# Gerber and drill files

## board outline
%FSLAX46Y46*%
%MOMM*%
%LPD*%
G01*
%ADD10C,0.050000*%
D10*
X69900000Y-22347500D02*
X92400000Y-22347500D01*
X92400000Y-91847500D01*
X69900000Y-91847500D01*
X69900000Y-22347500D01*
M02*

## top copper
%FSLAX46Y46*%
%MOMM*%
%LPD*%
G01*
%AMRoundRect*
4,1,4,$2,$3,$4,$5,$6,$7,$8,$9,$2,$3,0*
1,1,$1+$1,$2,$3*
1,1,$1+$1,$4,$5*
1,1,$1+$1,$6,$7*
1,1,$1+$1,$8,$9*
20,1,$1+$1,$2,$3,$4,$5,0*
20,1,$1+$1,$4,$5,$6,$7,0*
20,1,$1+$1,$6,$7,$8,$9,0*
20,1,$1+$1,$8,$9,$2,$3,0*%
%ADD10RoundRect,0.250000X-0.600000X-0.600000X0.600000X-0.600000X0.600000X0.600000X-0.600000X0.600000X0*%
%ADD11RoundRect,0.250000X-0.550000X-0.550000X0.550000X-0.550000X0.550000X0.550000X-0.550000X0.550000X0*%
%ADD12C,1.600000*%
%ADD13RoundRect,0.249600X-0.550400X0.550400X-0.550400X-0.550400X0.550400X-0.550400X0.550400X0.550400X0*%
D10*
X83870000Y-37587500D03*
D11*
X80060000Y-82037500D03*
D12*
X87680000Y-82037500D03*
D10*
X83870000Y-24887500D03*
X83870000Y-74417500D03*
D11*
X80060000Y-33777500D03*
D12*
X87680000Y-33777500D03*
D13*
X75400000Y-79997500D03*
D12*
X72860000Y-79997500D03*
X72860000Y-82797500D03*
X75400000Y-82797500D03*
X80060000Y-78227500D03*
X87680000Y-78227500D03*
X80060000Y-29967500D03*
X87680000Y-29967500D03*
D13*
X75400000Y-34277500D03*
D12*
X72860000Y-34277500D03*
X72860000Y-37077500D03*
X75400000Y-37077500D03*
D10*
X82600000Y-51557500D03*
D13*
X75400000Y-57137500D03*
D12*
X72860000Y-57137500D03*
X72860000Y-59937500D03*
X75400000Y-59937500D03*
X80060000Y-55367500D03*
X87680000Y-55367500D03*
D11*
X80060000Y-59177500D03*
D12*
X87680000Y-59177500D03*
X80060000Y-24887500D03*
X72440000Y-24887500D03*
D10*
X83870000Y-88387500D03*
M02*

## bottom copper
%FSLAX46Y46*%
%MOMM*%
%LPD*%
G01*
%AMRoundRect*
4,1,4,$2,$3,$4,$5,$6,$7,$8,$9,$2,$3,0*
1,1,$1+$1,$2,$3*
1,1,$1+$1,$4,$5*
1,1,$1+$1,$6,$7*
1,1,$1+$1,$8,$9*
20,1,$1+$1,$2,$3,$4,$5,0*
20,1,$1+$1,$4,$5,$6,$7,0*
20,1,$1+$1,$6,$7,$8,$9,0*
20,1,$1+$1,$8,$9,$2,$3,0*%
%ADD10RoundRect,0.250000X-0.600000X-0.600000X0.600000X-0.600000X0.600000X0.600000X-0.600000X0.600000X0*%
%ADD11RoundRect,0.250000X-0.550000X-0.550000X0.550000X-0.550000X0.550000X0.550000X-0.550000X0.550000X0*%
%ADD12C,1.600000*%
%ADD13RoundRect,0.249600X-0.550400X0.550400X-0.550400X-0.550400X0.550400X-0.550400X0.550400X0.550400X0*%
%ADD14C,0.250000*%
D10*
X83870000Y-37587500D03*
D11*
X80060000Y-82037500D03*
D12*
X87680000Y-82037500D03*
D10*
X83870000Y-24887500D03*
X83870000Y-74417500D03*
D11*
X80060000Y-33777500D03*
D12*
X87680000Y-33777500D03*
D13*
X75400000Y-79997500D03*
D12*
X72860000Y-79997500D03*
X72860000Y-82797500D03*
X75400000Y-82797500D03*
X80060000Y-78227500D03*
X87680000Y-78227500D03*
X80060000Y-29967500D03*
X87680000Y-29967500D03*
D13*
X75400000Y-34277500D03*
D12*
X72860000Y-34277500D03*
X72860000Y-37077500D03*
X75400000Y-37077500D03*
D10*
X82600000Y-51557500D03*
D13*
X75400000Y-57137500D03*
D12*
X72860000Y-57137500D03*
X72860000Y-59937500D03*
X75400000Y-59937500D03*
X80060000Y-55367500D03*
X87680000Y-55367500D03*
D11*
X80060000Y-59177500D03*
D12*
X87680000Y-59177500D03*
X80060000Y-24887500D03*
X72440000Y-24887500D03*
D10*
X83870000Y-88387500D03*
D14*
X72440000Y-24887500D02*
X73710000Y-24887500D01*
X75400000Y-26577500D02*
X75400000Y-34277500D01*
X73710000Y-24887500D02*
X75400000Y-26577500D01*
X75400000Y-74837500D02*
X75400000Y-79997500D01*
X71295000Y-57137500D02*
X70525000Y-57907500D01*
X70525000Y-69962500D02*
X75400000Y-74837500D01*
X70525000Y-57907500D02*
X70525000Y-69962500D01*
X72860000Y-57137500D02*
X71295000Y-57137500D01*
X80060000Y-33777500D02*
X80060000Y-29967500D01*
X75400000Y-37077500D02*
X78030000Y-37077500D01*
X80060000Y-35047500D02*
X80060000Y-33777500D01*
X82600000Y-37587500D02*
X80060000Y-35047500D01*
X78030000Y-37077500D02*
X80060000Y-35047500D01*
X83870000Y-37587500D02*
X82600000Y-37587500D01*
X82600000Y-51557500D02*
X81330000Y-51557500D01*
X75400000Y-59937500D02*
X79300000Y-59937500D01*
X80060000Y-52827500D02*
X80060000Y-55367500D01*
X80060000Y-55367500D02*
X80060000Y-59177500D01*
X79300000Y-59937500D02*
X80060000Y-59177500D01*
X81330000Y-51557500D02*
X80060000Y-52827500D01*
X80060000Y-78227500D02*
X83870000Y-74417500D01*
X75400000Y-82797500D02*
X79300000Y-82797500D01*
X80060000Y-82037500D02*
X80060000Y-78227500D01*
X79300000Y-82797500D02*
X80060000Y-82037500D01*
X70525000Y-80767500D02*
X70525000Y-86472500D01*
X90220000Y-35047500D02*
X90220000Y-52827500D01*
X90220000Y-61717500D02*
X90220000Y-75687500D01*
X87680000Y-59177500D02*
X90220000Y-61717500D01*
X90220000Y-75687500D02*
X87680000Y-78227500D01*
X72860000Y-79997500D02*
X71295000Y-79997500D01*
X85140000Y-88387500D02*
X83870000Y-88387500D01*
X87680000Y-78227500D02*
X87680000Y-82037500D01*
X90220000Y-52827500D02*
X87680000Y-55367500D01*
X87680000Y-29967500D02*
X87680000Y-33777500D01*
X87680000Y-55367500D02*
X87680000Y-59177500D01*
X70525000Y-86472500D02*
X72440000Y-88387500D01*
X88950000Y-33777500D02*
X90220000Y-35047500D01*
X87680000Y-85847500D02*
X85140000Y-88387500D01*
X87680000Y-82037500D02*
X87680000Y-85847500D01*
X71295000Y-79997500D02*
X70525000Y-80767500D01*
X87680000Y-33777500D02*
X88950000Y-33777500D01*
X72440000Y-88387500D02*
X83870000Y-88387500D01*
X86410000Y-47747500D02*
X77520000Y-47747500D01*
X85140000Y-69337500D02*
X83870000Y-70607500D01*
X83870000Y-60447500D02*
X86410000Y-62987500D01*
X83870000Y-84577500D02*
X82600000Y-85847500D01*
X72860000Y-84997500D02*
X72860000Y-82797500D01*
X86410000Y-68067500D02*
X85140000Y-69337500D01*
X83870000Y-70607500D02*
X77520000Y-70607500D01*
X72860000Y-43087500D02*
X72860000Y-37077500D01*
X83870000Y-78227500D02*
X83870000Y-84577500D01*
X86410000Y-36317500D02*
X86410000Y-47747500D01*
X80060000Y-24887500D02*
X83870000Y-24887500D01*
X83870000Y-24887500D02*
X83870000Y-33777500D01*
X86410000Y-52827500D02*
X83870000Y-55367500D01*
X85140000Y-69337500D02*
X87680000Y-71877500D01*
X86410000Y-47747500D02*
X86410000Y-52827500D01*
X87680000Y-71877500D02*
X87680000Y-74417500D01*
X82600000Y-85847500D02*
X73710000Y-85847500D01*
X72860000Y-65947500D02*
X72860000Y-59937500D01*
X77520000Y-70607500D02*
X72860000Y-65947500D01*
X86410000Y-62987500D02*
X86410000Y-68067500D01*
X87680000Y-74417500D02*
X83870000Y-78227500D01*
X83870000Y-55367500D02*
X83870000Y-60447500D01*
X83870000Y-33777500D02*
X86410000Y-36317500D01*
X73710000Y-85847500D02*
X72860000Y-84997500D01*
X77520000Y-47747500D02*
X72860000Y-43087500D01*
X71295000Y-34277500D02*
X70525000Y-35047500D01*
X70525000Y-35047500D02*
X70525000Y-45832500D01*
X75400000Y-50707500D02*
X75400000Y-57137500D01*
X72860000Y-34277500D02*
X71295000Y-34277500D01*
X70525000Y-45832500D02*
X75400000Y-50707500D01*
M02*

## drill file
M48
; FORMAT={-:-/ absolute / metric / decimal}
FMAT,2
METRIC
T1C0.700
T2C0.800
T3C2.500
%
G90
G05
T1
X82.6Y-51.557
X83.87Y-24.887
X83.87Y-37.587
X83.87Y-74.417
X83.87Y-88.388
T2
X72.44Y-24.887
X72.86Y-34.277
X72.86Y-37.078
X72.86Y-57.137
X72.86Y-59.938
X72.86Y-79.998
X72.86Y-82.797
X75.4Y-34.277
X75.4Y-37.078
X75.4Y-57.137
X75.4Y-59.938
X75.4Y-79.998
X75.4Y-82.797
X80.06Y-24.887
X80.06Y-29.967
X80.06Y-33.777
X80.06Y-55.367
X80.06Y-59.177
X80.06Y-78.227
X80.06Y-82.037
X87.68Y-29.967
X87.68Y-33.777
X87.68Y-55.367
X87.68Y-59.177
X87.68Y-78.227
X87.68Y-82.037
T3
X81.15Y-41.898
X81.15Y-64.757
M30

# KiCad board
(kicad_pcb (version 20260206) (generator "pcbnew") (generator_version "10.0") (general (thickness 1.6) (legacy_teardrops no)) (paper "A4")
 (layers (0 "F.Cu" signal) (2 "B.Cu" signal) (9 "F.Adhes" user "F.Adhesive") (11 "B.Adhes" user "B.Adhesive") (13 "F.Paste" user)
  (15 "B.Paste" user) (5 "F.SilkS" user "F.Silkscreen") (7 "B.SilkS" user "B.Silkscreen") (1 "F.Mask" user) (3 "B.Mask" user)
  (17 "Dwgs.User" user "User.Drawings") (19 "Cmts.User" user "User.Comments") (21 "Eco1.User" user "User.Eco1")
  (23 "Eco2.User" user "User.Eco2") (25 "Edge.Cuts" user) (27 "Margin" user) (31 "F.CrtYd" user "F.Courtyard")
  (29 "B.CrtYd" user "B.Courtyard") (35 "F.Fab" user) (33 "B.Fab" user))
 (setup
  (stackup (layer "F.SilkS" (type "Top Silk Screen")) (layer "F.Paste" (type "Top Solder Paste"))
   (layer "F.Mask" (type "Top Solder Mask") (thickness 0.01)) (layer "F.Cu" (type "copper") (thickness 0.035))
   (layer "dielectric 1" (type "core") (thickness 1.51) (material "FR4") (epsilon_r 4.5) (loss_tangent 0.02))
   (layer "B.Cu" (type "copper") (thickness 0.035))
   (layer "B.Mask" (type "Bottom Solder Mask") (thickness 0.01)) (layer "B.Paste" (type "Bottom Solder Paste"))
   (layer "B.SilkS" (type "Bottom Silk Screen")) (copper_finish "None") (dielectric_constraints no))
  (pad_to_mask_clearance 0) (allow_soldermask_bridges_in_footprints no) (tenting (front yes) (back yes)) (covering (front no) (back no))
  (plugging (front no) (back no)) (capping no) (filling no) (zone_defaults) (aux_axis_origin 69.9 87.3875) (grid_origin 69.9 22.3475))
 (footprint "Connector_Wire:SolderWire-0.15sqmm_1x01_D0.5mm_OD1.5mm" (layer "F.Cu") (at 83.87 37.5875)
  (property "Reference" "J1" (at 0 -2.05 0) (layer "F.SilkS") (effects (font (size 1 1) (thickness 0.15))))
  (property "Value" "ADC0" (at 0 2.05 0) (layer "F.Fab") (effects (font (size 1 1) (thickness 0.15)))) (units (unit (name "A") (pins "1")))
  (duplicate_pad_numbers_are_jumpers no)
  (pad "1" thru_hole roundrect (at 0 0) (size 1.7 1.7) (drill 0.7) (layers "*.Cu" "*.Mask") (remove_unused_layers no)
   (roundrect_rratio 0.147059) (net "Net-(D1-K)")))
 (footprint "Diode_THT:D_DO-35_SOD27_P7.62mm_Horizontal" (layer "F.Cu") (at 80.06 82.0375)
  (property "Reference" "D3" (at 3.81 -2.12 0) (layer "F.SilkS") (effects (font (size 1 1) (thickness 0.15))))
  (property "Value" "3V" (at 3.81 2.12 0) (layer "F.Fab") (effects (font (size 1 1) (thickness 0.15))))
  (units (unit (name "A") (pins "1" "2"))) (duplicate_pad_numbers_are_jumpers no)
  (pad "1" thru_hole roundrect (at 0 0) (size 1.6 1.6) (drill 0.8) (layers "*.Cu" "*.Mask") (remove_unused_layers no)
   (roundrect_rratio 0.15625) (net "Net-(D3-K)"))
  (pad "2" thru_hole circle (at 7.62 0) (size 1.6 1.6) (drill 0.8) (layers "*.Cu" "*.Mask") (remove_unused_layers no) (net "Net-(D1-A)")))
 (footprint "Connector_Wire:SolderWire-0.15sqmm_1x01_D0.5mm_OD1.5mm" (layer "F.Cu") (at 83.87 24.8875)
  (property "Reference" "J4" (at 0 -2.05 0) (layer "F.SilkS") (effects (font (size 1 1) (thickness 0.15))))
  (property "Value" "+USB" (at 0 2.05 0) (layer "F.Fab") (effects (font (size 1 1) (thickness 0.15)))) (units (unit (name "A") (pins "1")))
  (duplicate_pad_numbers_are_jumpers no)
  (pad "1" thru_hole roundrect (at 0 0) (size 1.7 1.7) (drill 0.7) (layers "*.Cu" "*.Mask") (remove_unused_layers no)
   (roundrect_rratio 0.147059) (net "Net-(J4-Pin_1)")))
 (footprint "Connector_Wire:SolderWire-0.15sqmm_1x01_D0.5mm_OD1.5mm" (layer "F.Cu") (at 83.87 74.4175)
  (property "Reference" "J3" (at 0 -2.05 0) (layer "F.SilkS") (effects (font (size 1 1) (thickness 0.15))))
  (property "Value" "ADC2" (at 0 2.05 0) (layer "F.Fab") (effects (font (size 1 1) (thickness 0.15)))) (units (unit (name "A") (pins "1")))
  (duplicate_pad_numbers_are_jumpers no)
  (pad "1" thru_hole roundrect (at 0 0) (size 1.7 1.7) (drill 0.7) (layers "*.Cu" "*.Mask") (remove_unused_layers no)
   (roundrect_rratio 0.147059) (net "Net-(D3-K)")))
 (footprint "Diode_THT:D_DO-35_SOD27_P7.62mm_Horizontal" (layer "F.Cu") (at 80.06 33.7775)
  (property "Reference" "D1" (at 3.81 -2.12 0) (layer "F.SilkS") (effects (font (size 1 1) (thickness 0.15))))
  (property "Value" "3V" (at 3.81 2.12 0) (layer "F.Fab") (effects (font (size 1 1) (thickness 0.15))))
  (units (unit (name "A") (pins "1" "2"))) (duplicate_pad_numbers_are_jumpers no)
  (pad "1" thru_hole roundrect (at 0 0) (size 1.6 1.6) (drill 0.8) (layers "*.Cu" "*.Mask") (remove_unused_layers no)
   (roundrect_rratio 0.15625) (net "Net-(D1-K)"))
  (pad "2" thru_hole circle (at 7.62 0) (size 1.6 1.6) (drill 0.8) (layers "*.Cu" "*.Mask") (remove_unused_layers no) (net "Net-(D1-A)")))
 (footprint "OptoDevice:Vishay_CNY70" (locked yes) (layer "F.Cu") (at 75.4 79.9975 -90)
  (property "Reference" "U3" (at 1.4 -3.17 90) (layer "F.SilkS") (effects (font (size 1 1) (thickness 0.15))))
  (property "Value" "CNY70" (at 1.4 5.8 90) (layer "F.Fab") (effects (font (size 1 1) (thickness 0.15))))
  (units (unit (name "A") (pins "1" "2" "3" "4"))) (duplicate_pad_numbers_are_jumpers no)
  (pad "1" thru_hole roundrect (at 0 0 270) (size 1.6 1.6) (drill 0.8) (layers "*.Cu" "*.Mask") (remove_unused_layers no)
   (roundrect_rratio 0.156) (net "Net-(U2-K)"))
  (pad "2" thru_hole circle (at 0 2.54 270) (size 1.6 1.6) (drill 0.8) (layers "*.Cu" "*.Mask") (remove_unused_layers no) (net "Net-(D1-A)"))
  (pad "3" thru_hole circle (at 2.8 2.54 270) (size 1.6 1.6) (drill 0.8) (layers "*.Cu" "*.Mask") (remove_unused_layers no)
   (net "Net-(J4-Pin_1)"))
  (pad "4" thru_hole circle (at 2.8 0 270) (size 1.6 1.6) (drill 0.8) (layers "*.Cu" "*.Mask") (remove_unused_layers no) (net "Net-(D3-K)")))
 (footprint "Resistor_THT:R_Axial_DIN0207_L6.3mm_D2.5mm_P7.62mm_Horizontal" (layer "F.Cu") (at 80.06 78.2275)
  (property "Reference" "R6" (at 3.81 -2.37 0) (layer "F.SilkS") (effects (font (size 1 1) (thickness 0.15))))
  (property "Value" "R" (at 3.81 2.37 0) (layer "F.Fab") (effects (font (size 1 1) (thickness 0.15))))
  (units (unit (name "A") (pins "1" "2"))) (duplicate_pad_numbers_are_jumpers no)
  (pad "1" thru_hole circle (at 0 0) (size 1.6 1.6) (drill 0.8) (layers "*.Cu" "*.Mask") (remove_unused_layers no) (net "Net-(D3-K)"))
  (pad "2" thru_hole circle (at 7.62 0) (size 1.6 1.6) (drill 0.8) (layers "*.Cu" "*.Mask") (remove_unused_layers no) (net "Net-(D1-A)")))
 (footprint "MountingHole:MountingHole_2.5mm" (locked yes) (layer "F.Cu") (at 81.15 41.8975)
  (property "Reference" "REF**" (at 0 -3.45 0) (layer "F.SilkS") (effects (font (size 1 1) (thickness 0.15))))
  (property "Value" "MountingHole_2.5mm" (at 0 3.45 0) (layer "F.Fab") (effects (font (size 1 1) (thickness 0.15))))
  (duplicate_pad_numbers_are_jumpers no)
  (pad "" np_thru_hole circle (at 0 0) (size 2.5 2.5) (drill 2.5) (layers "*.Mask" "B.Cu")))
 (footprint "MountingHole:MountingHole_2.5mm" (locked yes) (layer "F.Cu") (at 81.15 64.7575)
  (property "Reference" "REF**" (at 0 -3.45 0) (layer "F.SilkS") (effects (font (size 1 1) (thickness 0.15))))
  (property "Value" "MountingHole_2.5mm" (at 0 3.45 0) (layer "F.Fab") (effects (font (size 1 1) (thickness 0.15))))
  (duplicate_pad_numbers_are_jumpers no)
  (pad "" np_thru_hole circle (at 0 0) (size 2.5 2.5) (drill 2.5) (layers "*.Mask" "B.Cu")))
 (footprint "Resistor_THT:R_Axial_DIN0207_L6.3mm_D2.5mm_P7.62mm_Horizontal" (layer "F.Cu") (at 80.06 29.9675)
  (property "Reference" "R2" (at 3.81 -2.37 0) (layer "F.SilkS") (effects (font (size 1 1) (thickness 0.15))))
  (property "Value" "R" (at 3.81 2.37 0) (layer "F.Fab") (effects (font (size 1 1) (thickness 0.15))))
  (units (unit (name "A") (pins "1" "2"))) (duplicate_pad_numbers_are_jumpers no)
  (pad "1" thru_hole circle (at 0 0) (size 1.6 1.6) (drill 0.8) (layers "*.Cu" "*.Mask") (remove_unused_layers no) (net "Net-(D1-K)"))
  (pad "2" thru_hole circle (at 7.62 0) (size 1.6 1.6) (drill 0.8) (layers "*.Cu" "*.Mask") (remove_unused_layers no) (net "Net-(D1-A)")))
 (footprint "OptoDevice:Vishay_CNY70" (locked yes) (layer "F.Cu") (at 75.4 34.2775 -90)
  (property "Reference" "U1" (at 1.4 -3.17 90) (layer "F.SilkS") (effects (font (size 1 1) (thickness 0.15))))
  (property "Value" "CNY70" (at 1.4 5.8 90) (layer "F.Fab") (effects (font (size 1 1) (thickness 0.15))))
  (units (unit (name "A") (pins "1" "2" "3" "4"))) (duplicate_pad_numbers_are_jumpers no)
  (pad "1" thru_hole roundrect (at 0 0 270) (size 1.6 1.6) (drill 0.8) (layers "*.Cu" "*.Mask") (remove_unused_layers no)
   (roundrect_rratio 0.156) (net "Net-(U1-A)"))
  (pad "2" thru_hole circle (at 0 2.54 270) (size 1.6 1.6) (drill 0.8) (layers "*.Cu" "*.Mask") (remove_unused_layers no) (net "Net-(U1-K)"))
  (pad "3" thru_hole circle (at 2.8 2.54 270) (size 1.6 1.6) (drill 0.8) (layers "*.Cu" "*.Mask") (remove_unused_layers no)
   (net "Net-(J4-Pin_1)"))
  (pad "4" thru_hole circle (at 2.8 0 270) (size 1.6 1.6) (drill 0.8) (layers "*.Cu" "*.Mask") (remove_unused_layers no) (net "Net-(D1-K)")))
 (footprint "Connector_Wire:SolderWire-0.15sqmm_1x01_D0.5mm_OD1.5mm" (layer "F.Cu") (at 82.6 51.5575)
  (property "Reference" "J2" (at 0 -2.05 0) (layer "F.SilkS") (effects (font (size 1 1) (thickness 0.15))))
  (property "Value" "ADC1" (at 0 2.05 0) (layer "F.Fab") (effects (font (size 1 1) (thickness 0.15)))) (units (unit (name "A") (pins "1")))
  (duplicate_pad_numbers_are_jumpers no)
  (pad "1" thru_hole roundrect (at 0 0) (size 1.7 1.7) (drill 0.7) (layers "*.Cu" "*.Mask") (remove_unused_layers no)
   (roundrect_rratio 0.147059) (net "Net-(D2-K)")))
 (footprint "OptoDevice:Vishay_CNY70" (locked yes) (layer "F.Cu") (at 75.4 57.1375 -90)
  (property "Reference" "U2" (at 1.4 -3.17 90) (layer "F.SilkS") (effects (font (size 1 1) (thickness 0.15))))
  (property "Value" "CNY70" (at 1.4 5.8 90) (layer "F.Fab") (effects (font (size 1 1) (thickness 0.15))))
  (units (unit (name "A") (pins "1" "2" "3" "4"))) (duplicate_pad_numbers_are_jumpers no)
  (pad "1" thru_hole roundrect (at 0 0 270) (size 1.6 1.6) (drill 0.8) (layers "*.Cu" "*.Mask") (remove_unused_layers no)
   (roundrect_rratio 0.156) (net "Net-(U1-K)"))
  (pad "2" thru_hole circle (at 0 2.54 270) (size 1.6 1.6) (drill 0.8) (layers "*.Cu" "*.Mask") (remove_unused_layers no) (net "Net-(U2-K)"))
  (pad "3" thru_hole circle (at 2.8 2.54 270) (size 1.6 1.6) (drill 0.8) (layers "*.Cu" "*.Mask") (remove_unused_layers no)
   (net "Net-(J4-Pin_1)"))
  (pad "4" thru_hole circle (at 2.8 0 270) (size 1.6 1.6) (drill 0.8) (layers "*.Cu" "*.Mask") (remove_unused_layers no) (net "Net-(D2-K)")))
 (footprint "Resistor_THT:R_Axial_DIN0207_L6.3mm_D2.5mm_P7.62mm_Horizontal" (layer "F.Cu") (at 80.06 55.3675)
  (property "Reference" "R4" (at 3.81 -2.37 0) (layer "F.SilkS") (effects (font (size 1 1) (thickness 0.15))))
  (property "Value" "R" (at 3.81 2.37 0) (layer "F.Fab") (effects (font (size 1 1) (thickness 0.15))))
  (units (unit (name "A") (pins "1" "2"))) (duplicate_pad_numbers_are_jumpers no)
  (pad "1" thru_hole circle (at 0 0) (size 1.6 1.6) (drill 0.8) (layers "*.Cu" "*.Mask") (remove_unused_layers no) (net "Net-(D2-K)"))
  (pad "2" thru_hole circle (at 7.62 0) (size 1.6 1.6) (drill 0.8) (layers "*.Cu" "*.Mask") (remove_unused_layers no) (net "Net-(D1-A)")))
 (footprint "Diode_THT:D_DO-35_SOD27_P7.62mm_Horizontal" (layer "F.Cu") (at 80.06 59.1775)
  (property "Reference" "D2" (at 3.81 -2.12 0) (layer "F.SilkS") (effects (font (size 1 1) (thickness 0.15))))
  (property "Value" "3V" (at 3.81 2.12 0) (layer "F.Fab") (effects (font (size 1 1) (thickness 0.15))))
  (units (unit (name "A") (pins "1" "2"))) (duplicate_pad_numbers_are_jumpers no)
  (pad "1" thru_hole roundrect (at 0 0) (size 1.6 1.6) (drill 0.8) (layers "*.Cu" "*.Mask") (remove_unused_layers no)
   (roundrect_rratio 0.15625) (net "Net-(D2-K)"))
  (pad "2" thru_hole circle (at 7.62 0) (size 1.6 1.6) (drill 0.8) (layers "*.Cu" "*.Mask") (remove_unused_layers no) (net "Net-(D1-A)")))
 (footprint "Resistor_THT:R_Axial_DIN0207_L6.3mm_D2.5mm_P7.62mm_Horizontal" (layer "F.Cu") (at 80.06 24.8875 180)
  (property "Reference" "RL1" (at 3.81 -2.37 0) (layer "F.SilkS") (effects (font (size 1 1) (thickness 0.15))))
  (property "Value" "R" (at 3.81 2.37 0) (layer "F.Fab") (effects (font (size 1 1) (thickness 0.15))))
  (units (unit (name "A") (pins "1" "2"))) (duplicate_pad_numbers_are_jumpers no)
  (pad "1" thru_hole circle (at 0 0 180) (size 1.6 1.6) (drill 0.8) (layers "*.Cu" "*.Mask") (remove_unused_layers no)
   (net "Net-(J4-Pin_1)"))
  (pad "2" thru_hole circle (at 7.62 0 180) (size 1.6 1.6) (drill 0.8) (layers "*.Cu" "*.Mask") (remove_unused_layers no) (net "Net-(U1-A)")))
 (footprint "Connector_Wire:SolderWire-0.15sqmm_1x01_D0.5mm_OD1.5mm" (layer "F.Cu") (at 83.87 88.3875)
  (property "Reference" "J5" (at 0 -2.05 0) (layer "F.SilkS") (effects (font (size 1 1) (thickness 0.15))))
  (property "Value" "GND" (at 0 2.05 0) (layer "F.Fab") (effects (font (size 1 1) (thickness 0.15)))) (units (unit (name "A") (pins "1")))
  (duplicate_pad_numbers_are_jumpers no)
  (pad "1" thru_hole roundrect (at 0 0) (size 1.7 1.7) (drill 0.7) (layers "*.Cu" "*.Mask") (remove_unused_layers no)
   (roundrect_rratio 0.147059) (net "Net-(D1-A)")))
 (gr_rect (start 69.9 22.3475) (end 92.4 91.8475) (stroke (width 0.05) (type solid)) (fill no) (layer "Edge.Cuts"))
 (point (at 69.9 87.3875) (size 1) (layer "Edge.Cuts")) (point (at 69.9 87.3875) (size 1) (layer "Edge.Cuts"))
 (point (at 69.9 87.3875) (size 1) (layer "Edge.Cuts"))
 (segment (start 72.44 24.8875) (end 73.71 24.8875) (width 0.25) (layer "B.Cu") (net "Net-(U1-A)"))
 (segment (start 75.4 26.5775) (end 75.4 34.2775) (width 0.25) (layer "B.Cu") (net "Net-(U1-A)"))
 (segment (start 73.71 24.8875) (end 75.4 26.5775) (width 0.25) (layer "B.Cu") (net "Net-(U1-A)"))
 (segment (start 75.4 74.8375) (end 75.4 79.9975) (width 0.25) (layer "B.Cu") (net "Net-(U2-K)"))
 (segment (start 71.295 57.1375) (end 70.525 57.9075) (width 0.25) (layer "B.Cu") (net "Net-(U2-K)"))
 (segment (start 70.525 69.9625) (end 75.4 74.8375) (width 0.25) (layer "B.Cu") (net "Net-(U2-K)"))
 (segment (start 70.525 57.9075) (end 70.525 69.9625) (width 0.25) (layer "B.Cu") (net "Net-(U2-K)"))
 (segment (start 72.86 57.1375) (end 71.295 57.1375) (width 0.25) (layer "B.Cu") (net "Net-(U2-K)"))
 (segment (start 80.06 33.7775) (end 80.06 29.9675) (width 0.25) (layer "B.Cu") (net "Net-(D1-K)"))
 (segment (start 75.4 37.0775) (end 78.03 37.0775) (width 0.25) (layer "B.Cu") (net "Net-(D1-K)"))
 (segment (start 80.06 35.0475) (end 80.06 33.7775) (width 0.25) (layer "B.Cu") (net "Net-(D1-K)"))
 (segment (start 82.6 37.5875) (end 80.06 35.0475) (width 0.25) (layer "B.Cu") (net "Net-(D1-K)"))
 (segment (start 78.03 37.0775) (end 80.06 35.0475) (width 0.25) (layer "B.Cu") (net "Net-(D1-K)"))
 (segment (start 83.87 37.5875) (end 82.6 37.5875) (width 0.25) (layer "B.Cu") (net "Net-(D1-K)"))
 (segment (start 82.6 51.5575) (end 81.33 51.5575) (width 0.25) (layer "B.Cu") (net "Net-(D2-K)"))
 (segment (start 75.4 59.9375) (end 79.3 59.9375) (width 0.25) (layer "B.Cu") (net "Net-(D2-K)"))
 (segment (start 80.06 52.8275) (end 80.06 55.3675) (width 0.25) (layer "B.Cu") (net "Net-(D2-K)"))
 (segment (start 80.06 55.3675) (end 80.06 59.1775) (width 0.25) (layer "B.Cu") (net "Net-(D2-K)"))
 (segment (start 79.3 59.9375) (end 80.06 59.1775) (width 0.25) (layer "B.Cu") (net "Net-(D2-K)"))
 (segment (start 81.33 51.5575) (end 80.06 52.8275) (width 0.25) (layer "B.Cu") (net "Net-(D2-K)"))
 (segment (start 80.06 78.2275) (end 83.87 74.4175) (width 0.25) (layer "B.Cu") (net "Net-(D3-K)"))
 (segment (start 75.4 82.7975) (end 79.3 82.7975) (width 0.25) (layer "B.Cu") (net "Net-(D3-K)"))
 (segment (start 80.06 82.0375) (end 80.06 78.2275) (width 0.25) (layer "B.Cu") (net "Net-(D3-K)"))
 (segment (start 79.3 82.7975) (end 80.06 82.0375) (width 0.25) (layer "B.Cu") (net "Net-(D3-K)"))
 (segment (start 70.525 80.7675) (end 70.525 86.4725) (width 0.25) (layer "B.Cu") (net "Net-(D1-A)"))
 (segment (start 90.22 35.0475) (end 90.22 52.8275) (width 0.25) (layer "B.Cu") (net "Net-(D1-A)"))
 (segment (start 90.22 61.7175) (end 90.22 75.6875) (width 0.25) (layer "B.Cu") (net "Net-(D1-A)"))
 (segment (start 87.68 59.1775) (end 90.22 61.7175) (width 0.25) (layer "B.Cu") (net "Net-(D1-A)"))
 (segment (start 90.22 75.6875) (end 87.68 78.2275) (width 0.25) (layer "B.Cu") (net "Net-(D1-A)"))
 (segment (start 72.86 79.9975) (end 71.295 79.9975) (width 0.25) (layer "B.Cu") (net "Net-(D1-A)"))
 (segment (start 85.14 88.3875) (end 83.87 88.3875) (width 0.25) (layer "B.Cu") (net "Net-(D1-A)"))
 (segment (start 87.68 78.2275) (end 87.68 82.0375) (width 0.25) (layer "B.Cu") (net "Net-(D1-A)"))
 (segment (start 90.22 52.8275) (end 87.68 55.3675) (width 0.25) (layer "B.Cu") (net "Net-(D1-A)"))
 (segment (start 87.68 29.9675) (end 87.68 33.7775) (width 0.25) (layer "B.Cu") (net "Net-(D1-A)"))
 (segment (start 87.68 55.3675) (end 87.68 59.1775) (width 0.25) (layer "B.Cu") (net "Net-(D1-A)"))
 (segment (start 70.525 86.4725) (end 72.44 88.3875) (width 0.25) (layer "B.Cu") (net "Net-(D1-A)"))
 (segment (start 88.95 33.7775) (end 90.22 35.0475) (width 0.25) (layer "B.Cu") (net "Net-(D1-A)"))
 (segment (start 87.68 85.8475) (end 85.14 88.3875) (width 0.25) (layer "B.Cu") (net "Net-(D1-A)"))
 (segment (start 87.68 82.0375) (end 87.68 85.8475) (width 0.25) (layer "B.Cu") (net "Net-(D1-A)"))
 (segment (start 71.295 79.9975) (end 70.525 80.7675) (width 0.25) (layer "B.Cu") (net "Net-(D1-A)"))
 (segment (start 87.68 33.7775) (end 88.95 33.7775) (width 0.25) (layer "B.Cu") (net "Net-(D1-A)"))
 (segment (start 72.44 88.3875) (end 83.87 88.3875) (width 0.25) (layer "B.Cu") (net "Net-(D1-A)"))
 (segment (start 86.41 47.7475) (end 77.52 47.7475) (width 0.25) (layer "B.Cu") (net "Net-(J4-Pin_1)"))
 (segment (start 85.14 69.3375) (end 83.87 70.6075) (width 0.25) (layer "B.Cu") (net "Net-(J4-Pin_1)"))
 (segment (start 83.87 60.4475) (end 86.41 62.9875) (width 0.25) (layer "B.Cu") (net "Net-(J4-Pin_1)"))
 (segment (start 83.87 84.5775) (end 82.6 85.8475) (width 0.25) (layer "B.Cu") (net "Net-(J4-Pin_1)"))
 (segment (start 72.86 84.9975) (end 72.86 82.7975) (width 0.25) (layer "B.Cu") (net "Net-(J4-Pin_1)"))
 (segment (start 86.41 68.0675) (end 85.14 69.3375) (width 0.25) (layer "B.Cu") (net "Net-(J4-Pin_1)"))
 (segment (start 83.87 70.6075) (end 77.52 70.6075) (width 0.25) (layer "B.Cu") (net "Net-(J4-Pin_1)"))
 (segment (start 72.86 43.0875) (end 72.86 37.0775) (width 0.25) (layer "B.Cu") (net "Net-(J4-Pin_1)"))
 (segment (start 83.87 78.2275) (end 83.87 84.5775) (width 0.25) (layer "B.Cu") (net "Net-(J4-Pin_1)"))
 (segment (start 86.41 36.3175) (end 86.41 47.7475) (width 0.25) (layer "B.Cu") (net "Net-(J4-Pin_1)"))
 (segment (start 80.06 24.8875) (end 83.87 24.8875) (width 0.25) (layer "B.Cu") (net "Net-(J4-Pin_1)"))
 (segment (start 83.87 24.8875) (end 83.87 33.7775) (width 0.25) (layer "B.Cu") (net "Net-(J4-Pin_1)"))
 (segment (start 86.41 52.8275) (end 83.87 55.3675) (width 0.25) (layer "B.Cu") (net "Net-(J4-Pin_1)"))
 (segment (start 85.14 69.3375) (end 87.68 71.8775) (width 0.25) (layer "B.Cu") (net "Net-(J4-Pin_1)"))
 (segment (start 86.41 47.7475) (end 86.41 52.8275) (width 0.25) (layer "B.Cu") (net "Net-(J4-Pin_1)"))
 (segment (start 87.68 71.8775) (end 87.68 74.4175) (width 0.25) (layer "B.Cu") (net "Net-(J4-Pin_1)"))
 (segment (start 82.6 85.8475) (end 73.71 85.8475) (width 0.25) (layer "B.Cu") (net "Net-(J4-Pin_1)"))
 (segment (start 72.86 65.9475) (end 72.86 59.9375) (width 0.25) (layer "B.Cu") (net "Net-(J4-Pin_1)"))
 (segment (start 77.52 70.6075) (end 72.86 65.9475) (width 0.25) (layer "B.Cu") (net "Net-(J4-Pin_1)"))
 (segment (start 86.41 62.9875) (end 86.41 68.0675) (width 0.25) (layer "B.Cu") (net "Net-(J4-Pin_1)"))
 (segment (start 87.68 74.4175) (end 83.87 78.2275) (width 0.25) (layer "B.Cu") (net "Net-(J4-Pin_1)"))
 (segment (start 83.87 55.3675) (end 83.87 60.4475) (width 0.25) (layer "B.Cu") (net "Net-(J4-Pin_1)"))
 (segment (start 83.87 33.7775) (end 86.41 36.3175) (width 0.25) (layer "B.Cu") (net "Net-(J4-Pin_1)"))
 (segment (start 73.71 85.8475) (end 72.86 84.9975) (width 0.25) (layer "B.Cu") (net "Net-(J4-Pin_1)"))
 (segment (start 77.52 47.7475) (end 72.86 43.0875) (width 0.25) (layer "B.Cu") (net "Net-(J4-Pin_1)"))
 (segment (start 71.295 34.2775) (end 70.525 35.0475) (width 0.25) (layer "B.Cu") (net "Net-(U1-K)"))
 (segment (start 70.525 35.0475) (end 70.525 45.8325) (width 0.25) (layer "B.Cu") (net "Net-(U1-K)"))
 (segment (start 75.4 50.7075) (end 75.4 57.1375) (width 0.25) (layer "B.Cu") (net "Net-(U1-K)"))
 (segment (start 72.86 34.2775) (end 71.295 34.2775) (width 0.25) (layer "B.Cu") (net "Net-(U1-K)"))
 (segment (start 70.525 45.8325) (end 75.4 50.7075) (width 0.25) (layer "B.Cu") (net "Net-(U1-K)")))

